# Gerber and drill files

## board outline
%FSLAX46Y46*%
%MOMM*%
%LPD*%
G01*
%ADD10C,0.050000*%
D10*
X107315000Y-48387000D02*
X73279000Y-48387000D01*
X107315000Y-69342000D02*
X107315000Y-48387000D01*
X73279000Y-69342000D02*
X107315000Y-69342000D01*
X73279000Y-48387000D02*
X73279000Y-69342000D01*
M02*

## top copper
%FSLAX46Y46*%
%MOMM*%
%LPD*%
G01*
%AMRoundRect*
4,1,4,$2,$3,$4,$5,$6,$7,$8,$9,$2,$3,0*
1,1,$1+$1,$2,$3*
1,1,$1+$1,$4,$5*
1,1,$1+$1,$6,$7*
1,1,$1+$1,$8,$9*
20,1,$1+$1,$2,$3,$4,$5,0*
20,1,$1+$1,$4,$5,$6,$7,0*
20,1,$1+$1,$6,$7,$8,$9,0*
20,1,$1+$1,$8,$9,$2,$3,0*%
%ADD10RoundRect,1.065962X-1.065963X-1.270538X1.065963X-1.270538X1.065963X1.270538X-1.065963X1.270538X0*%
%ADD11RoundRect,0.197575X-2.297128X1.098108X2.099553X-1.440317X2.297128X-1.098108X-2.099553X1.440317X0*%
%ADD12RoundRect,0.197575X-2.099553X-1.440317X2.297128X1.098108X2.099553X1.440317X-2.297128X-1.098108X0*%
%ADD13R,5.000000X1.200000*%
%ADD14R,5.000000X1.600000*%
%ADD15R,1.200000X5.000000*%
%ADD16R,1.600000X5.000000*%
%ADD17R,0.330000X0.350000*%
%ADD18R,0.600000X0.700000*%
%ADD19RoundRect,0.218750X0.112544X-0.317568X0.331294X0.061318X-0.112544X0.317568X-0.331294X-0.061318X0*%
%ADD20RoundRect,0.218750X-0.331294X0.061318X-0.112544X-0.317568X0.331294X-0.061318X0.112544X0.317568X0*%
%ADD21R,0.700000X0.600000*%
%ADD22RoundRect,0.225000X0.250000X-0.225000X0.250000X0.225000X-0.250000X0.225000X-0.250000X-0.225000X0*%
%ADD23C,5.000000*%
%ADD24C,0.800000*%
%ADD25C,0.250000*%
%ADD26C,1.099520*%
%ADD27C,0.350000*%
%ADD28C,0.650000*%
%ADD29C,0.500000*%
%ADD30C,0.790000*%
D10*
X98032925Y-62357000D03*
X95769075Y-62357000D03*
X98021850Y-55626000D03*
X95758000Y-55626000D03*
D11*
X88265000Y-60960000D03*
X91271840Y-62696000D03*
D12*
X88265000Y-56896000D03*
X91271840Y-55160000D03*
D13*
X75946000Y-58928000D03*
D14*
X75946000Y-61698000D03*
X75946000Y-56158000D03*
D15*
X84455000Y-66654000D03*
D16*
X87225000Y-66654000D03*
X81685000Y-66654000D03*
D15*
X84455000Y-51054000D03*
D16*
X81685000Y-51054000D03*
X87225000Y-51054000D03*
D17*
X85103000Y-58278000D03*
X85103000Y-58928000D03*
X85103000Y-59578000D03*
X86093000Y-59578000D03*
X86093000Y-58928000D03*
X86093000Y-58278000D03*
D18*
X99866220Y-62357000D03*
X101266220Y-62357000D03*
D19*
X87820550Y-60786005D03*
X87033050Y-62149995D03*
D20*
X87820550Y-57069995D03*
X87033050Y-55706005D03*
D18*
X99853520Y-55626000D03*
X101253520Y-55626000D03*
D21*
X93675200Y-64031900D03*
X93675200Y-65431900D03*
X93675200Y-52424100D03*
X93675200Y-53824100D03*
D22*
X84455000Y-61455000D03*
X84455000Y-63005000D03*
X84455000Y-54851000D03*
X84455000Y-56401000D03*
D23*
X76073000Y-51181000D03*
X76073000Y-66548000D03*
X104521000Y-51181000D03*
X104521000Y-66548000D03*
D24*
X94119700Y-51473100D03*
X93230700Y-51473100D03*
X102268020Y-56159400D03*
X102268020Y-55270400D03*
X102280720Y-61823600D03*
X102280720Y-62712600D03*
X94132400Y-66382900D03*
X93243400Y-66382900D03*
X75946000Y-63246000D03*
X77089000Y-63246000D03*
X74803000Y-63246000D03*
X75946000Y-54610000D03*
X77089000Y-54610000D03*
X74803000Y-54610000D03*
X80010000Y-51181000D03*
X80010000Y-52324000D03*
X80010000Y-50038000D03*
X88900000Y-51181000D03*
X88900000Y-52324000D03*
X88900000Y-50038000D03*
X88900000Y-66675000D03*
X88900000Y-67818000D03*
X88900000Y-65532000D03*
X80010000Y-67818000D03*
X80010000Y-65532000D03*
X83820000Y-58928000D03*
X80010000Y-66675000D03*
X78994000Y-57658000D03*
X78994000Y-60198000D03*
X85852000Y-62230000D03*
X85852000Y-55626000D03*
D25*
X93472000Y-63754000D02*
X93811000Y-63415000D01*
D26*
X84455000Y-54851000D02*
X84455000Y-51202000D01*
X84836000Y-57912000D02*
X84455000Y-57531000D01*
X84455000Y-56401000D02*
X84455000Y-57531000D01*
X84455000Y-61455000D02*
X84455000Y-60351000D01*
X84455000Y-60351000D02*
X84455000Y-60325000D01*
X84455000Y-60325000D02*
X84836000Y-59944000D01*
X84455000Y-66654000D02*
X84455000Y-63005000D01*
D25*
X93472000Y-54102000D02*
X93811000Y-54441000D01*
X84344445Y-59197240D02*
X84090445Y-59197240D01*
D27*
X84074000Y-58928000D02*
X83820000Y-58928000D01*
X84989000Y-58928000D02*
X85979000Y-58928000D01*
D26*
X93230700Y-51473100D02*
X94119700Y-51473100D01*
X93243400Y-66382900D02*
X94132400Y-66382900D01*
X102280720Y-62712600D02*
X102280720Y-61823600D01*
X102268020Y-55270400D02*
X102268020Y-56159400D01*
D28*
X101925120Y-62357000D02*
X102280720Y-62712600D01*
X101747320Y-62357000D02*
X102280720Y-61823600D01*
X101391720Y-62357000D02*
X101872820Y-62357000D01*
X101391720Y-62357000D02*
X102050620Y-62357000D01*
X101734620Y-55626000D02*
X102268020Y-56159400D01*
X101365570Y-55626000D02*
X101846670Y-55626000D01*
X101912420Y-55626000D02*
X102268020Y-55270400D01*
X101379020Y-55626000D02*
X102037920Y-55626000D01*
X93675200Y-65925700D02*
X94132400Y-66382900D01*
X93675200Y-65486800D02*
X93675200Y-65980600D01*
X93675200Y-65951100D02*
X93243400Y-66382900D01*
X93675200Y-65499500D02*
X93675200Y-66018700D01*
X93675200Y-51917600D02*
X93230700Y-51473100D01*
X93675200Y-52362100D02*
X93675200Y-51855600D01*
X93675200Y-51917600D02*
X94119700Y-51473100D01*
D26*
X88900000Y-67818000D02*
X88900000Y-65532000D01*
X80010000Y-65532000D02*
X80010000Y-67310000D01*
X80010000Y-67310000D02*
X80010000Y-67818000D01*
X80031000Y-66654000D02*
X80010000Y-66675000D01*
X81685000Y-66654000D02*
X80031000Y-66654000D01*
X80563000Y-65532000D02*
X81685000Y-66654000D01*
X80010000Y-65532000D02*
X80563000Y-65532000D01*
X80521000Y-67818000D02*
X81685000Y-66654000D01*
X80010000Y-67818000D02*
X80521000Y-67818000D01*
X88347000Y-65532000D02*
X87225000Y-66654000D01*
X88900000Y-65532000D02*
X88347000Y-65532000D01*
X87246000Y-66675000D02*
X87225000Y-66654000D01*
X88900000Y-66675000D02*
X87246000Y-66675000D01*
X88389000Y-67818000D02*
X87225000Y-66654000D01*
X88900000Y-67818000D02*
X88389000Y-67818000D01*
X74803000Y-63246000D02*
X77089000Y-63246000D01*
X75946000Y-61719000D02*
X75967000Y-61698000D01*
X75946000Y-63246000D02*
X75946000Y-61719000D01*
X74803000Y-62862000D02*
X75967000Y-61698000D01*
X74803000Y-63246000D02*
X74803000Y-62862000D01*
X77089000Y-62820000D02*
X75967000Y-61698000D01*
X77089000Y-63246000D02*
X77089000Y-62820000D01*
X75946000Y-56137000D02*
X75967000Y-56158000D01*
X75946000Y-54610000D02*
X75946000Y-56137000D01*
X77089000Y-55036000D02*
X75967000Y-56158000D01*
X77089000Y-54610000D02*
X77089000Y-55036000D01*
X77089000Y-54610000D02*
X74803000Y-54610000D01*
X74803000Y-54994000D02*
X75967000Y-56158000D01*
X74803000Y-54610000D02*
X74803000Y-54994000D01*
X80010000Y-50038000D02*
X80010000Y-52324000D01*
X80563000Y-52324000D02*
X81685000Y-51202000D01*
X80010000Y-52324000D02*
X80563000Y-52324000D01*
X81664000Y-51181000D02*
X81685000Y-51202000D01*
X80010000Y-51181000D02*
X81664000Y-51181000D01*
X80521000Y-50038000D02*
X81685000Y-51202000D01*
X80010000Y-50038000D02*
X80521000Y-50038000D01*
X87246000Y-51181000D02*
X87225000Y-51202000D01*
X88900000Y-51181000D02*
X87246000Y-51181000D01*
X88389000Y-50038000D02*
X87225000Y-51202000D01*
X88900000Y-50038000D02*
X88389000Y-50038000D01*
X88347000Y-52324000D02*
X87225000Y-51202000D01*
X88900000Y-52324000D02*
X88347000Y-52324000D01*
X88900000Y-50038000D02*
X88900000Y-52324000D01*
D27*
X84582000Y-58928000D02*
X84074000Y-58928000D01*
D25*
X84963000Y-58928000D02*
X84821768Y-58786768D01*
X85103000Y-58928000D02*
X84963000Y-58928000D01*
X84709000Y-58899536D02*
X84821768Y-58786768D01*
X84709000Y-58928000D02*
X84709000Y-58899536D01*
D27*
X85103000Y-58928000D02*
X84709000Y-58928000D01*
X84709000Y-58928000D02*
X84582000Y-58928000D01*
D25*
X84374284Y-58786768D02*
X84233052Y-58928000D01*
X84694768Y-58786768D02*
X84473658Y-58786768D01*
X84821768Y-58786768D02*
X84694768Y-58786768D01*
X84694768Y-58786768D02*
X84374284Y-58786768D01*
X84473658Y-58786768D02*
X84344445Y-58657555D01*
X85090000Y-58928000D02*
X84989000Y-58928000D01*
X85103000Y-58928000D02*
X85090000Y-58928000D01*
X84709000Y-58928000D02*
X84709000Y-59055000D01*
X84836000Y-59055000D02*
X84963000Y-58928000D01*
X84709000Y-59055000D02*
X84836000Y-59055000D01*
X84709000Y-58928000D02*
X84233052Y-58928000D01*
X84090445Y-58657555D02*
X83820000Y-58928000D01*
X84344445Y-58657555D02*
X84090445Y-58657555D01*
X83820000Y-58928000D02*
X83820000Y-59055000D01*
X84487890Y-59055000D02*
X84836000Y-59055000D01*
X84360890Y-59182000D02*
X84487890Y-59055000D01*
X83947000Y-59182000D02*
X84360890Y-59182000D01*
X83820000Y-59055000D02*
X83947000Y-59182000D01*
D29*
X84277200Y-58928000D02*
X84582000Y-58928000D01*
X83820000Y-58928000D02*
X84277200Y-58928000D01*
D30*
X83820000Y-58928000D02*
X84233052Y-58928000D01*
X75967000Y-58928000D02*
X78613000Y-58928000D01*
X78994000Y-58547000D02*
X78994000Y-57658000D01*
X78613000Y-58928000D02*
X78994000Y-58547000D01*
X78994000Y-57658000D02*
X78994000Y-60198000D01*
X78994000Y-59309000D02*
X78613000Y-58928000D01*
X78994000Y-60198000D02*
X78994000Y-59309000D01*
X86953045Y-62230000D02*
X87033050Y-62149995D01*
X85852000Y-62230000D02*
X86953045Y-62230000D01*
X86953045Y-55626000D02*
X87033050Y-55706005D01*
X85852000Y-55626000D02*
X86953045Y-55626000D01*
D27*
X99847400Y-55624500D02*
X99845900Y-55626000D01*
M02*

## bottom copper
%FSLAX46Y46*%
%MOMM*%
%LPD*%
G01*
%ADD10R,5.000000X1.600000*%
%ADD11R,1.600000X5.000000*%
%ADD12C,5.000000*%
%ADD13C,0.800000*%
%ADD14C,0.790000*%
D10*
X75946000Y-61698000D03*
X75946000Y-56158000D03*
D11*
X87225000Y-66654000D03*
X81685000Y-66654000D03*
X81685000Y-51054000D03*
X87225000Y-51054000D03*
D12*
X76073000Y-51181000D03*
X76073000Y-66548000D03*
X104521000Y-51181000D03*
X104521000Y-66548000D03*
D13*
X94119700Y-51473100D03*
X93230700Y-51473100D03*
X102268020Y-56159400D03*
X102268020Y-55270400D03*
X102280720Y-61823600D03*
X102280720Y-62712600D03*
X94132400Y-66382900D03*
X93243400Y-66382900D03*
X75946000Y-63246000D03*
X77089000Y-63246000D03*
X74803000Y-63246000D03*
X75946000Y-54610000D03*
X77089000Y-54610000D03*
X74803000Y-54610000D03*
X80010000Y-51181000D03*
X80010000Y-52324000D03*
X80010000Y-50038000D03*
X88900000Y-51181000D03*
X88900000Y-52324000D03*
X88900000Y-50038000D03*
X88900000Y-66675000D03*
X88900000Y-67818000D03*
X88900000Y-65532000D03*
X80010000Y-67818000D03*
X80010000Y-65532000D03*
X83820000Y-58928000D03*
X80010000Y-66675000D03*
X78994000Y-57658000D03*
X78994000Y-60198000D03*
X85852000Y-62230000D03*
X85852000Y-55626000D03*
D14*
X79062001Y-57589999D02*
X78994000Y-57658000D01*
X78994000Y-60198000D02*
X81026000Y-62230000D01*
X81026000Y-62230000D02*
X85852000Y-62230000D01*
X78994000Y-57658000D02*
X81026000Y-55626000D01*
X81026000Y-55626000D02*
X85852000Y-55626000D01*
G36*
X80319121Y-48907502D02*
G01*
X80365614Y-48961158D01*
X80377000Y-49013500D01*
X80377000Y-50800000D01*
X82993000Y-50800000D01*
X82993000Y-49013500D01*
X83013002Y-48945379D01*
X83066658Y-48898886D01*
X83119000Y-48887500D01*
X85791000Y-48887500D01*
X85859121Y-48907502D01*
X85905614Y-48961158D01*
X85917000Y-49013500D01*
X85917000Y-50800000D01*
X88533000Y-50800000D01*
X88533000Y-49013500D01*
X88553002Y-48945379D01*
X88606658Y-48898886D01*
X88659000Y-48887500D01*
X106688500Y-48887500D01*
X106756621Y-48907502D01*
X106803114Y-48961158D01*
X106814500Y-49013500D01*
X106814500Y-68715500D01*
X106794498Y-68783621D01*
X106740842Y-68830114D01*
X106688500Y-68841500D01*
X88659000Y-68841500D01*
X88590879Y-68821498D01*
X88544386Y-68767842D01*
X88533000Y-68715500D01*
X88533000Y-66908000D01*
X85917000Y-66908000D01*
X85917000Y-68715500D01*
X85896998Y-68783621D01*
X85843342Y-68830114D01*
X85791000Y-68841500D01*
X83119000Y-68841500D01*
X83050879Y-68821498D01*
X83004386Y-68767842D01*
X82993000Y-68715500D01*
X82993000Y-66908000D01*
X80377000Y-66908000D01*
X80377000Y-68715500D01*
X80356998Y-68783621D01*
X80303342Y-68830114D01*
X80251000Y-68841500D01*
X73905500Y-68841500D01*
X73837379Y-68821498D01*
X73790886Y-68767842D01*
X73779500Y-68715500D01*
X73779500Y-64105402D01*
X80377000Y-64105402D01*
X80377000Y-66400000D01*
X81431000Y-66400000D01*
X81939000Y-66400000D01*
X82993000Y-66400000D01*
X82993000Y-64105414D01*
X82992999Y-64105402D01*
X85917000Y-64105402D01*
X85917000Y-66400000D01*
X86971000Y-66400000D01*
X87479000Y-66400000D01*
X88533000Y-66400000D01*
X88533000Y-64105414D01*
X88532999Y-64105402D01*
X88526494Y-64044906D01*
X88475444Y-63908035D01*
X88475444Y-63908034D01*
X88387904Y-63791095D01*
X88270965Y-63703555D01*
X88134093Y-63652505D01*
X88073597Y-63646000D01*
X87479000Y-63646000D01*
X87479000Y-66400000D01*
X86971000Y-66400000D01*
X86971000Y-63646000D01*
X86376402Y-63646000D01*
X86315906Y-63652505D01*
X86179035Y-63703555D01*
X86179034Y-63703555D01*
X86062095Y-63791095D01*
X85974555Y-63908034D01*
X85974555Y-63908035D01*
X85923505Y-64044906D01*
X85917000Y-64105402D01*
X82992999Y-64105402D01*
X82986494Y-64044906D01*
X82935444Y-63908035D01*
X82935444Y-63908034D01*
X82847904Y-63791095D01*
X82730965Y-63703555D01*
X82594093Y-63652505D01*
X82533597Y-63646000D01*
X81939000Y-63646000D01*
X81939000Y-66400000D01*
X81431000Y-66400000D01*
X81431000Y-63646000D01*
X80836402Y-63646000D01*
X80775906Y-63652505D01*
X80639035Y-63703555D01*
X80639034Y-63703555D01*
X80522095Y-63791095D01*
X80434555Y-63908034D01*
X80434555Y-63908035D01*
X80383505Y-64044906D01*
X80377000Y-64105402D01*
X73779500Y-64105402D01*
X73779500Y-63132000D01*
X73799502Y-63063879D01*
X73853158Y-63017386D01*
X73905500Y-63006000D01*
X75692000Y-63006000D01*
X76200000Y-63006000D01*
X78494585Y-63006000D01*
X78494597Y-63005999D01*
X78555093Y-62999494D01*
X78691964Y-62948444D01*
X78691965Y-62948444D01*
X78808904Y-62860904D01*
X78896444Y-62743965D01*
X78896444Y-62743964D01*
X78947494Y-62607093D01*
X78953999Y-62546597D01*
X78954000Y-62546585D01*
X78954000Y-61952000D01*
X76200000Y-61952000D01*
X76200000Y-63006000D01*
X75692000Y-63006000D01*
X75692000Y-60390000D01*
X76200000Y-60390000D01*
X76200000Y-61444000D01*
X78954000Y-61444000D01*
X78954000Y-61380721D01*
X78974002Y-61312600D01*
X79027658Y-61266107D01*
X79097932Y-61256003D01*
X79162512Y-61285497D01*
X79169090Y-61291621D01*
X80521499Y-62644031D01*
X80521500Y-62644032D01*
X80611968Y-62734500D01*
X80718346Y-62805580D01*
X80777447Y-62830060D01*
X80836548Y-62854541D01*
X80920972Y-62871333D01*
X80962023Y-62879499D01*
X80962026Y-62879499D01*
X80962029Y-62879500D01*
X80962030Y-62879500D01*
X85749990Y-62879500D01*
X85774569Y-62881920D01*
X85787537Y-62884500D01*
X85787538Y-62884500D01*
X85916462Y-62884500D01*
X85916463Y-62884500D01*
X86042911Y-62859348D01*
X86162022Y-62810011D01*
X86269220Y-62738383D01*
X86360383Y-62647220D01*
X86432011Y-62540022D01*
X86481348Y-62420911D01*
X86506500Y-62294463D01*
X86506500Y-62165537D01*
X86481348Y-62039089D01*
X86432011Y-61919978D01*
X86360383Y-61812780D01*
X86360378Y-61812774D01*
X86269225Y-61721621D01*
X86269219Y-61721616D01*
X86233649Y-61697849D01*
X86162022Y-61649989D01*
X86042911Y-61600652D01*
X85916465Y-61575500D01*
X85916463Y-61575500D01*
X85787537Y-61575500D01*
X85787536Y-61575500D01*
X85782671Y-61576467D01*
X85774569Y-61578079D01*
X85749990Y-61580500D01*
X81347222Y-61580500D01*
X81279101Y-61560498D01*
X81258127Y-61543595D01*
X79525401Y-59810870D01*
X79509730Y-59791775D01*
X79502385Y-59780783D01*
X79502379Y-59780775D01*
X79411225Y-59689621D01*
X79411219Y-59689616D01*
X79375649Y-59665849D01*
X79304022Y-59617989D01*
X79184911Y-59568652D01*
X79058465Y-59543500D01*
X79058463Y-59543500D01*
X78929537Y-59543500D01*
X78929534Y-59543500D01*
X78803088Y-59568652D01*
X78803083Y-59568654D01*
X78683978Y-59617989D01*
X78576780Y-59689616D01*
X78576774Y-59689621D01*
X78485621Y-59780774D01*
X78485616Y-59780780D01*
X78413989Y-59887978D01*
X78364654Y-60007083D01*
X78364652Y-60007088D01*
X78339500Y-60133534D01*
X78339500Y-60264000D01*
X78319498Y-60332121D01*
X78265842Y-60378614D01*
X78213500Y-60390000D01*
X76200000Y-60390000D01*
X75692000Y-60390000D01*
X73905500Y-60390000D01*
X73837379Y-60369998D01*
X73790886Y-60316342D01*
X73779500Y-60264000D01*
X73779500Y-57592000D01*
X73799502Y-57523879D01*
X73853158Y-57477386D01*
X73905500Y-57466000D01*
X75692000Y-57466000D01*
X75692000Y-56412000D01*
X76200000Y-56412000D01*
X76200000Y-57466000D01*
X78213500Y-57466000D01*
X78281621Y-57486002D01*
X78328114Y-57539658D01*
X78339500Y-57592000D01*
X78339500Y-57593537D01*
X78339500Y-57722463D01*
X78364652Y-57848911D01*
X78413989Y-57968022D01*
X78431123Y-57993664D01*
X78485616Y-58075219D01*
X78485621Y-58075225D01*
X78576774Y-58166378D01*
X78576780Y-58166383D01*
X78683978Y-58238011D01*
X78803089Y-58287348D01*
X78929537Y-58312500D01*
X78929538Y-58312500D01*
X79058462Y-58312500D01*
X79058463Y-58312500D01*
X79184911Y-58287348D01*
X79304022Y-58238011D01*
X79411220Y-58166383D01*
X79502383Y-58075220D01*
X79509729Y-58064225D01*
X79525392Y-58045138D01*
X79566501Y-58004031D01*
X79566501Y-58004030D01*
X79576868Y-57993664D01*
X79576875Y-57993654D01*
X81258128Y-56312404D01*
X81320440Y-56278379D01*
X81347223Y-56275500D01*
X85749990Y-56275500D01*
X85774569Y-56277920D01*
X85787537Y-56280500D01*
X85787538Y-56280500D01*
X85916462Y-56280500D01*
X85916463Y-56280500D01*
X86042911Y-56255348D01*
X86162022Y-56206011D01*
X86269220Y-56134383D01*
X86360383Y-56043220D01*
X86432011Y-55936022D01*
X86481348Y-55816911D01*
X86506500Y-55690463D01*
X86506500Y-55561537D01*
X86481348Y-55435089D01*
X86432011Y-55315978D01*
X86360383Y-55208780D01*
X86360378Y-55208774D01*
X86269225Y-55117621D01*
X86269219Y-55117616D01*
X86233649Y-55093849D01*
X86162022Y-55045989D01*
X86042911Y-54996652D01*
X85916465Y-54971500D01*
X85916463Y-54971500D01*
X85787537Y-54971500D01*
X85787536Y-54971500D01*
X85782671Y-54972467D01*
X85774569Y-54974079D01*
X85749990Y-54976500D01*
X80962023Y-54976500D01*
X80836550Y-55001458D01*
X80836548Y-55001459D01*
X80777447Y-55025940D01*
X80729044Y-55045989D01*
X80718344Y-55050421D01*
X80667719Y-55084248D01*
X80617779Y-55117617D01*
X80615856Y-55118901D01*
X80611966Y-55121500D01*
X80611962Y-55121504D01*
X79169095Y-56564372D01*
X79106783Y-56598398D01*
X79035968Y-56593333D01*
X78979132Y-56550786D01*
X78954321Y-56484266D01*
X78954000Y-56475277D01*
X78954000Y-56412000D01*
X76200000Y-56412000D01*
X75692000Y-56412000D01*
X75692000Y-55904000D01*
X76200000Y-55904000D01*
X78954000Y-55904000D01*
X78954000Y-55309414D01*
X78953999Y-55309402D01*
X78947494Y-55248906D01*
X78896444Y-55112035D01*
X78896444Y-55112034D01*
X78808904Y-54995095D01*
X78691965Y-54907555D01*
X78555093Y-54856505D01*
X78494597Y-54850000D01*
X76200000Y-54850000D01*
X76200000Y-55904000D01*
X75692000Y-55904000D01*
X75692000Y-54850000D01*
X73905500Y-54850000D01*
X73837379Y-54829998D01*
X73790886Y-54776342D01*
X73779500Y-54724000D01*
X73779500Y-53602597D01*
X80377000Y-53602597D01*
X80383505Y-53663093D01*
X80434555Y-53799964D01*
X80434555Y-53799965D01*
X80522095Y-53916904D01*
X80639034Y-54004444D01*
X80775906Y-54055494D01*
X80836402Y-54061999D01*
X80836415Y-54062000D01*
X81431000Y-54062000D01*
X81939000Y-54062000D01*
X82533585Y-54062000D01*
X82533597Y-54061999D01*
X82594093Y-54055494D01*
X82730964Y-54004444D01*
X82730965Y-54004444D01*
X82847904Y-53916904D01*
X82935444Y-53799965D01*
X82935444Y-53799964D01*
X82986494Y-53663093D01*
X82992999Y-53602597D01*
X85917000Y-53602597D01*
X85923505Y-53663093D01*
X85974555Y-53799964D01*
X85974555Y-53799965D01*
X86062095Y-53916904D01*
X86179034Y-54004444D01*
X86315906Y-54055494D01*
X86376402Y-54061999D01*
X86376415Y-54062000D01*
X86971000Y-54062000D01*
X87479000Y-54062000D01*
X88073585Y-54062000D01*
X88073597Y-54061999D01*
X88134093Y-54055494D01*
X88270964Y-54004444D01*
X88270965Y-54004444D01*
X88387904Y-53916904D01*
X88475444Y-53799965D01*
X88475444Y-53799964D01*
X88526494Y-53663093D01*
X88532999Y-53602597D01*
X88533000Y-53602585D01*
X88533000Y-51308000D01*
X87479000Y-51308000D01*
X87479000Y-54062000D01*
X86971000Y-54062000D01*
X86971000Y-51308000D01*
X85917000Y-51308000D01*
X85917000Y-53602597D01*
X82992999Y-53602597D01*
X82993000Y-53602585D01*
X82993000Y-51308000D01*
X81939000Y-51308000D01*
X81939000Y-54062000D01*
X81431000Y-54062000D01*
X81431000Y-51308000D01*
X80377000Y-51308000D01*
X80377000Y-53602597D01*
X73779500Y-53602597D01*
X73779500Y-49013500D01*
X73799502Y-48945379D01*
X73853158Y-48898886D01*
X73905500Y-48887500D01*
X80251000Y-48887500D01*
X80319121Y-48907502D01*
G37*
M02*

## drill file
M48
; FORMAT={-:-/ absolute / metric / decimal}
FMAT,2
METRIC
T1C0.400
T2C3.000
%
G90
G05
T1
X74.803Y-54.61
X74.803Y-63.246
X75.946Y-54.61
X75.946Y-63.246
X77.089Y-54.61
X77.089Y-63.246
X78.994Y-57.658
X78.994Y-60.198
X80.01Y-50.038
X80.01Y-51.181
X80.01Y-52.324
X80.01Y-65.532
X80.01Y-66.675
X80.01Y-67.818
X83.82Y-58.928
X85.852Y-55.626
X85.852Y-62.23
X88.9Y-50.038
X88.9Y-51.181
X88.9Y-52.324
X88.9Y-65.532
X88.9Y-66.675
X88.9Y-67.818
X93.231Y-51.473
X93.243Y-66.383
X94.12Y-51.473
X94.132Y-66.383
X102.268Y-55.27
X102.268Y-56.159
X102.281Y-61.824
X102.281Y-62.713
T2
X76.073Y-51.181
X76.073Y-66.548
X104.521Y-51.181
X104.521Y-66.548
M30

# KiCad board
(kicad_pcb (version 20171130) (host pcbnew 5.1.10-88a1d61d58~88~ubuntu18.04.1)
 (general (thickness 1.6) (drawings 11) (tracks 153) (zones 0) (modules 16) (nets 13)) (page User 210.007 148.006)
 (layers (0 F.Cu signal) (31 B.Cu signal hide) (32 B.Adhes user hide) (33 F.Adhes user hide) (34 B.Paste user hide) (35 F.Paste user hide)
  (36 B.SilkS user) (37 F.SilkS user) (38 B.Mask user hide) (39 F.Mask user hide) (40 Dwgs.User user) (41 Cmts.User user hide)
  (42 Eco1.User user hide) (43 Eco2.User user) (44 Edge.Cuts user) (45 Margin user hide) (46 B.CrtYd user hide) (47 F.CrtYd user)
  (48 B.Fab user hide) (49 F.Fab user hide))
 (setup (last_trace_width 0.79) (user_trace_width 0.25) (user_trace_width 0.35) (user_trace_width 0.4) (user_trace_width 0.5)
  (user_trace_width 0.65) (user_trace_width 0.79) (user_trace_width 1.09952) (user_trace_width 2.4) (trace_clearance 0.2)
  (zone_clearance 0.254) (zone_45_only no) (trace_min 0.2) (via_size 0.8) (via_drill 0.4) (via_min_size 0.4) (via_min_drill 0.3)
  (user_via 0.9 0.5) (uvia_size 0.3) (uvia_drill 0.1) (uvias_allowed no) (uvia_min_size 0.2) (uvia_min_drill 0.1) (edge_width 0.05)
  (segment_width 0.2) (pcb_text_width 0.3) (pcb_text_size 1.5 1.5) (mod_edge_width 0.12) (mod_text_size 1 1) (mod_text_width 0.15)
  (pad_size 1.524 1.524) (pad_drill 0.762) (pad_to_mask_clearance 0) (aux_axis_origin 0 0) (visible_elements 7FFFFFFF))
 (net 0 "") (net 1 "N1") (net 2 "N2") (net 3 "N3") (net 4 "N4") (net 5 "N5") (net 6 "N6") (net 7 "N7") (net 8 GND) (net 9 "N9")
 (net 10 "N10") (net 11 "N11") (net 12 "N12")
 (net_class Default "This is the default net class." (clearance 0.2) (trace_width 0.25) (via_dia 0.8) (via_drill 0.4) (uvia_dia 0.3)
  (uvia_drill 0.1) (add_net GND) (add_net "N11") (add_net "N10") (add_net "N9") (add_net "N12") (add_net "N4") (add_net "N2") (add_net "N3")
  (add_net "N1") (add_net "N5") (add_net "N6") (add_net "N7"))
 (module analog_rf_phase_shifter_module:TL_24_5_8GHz (layer F.Cu) (at 96.901 62.357)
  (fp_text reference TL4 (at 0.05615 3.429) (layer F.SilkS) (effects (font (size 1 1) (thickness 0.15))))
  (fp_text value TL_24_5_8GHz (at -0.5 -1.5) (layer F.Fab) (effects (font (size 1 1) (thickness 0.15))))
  (pad 2 smd roundrect (at 1.131925 0) (size 4.26385 4.673) (layers F.Cu) (roundrect_rratio 0.2499998827350868) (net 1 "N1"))
  (pad 1 smd roundrect (at -1.131925 0) (size 4.26385 4.673) (layers F.Cu) (roundrect_rratio 0.2499998827350868) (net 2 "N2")))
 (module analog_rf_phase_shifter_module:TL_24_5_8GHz (layer F.Cu) (at 96.889925 55.626)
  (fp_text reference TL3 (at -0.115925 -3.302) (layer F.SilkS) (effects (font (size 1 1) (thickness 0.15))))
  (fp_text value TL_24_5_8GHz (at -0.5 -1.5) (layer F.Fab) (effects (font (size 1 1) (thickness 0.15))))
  (pad 2 smd roundrect (at 1.131925 0) (size 4.26385 4.673) (layers F.Cu) (roundrect_rratio 0.2499998827350868) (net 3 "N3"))
  (pad 1 smd roundrect (at -1.131925 0) (size 4.26385 4.673) (layers F.Cu) (roundrect_rratio 0.2499998827350868) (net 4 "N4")))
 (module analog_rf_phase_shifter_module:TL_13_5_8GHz (layer F.Cu) (at 89.76842 61.828 330)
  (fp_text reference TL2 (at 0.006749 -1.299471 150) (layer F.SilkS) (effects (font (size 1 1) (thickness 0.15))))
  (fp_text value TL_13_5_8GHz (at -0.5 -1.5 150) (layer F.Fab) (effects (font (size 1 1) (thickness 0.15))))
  (pad 1 smd roundrect (at -1.736 0 330) (size 5.472 0.7903) (layers F.Cu) (roundrect_rratio 0.25) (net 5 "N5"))
  (pad 2 smd roundrect (at 1.736 0 330) (size 5.472 0.7903) (layers F.Cu) (roundrect_rratio 0.25) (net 2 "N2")))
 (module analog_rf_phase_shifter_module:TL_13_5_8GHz (layer F.Cu) (at 89.76842 56.028 30)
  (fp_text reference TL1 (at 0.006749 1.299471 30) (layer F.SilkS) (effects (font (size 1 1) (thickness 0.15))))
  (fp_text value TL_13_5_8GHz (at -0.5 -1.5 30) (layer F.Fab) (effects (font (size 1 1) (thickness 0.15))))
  (pad 1 smd roundrect (at -1.736 0 30) (size 5.472 0.7903) (layers F.Cu) (roundrect_rratio 0.25) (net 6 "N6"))
  (pad 2 smd roundrect (at 1.736 0 30) (size 5.472 0.7903) (layers F.Cu) (roundrect_rratio 0.25) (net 4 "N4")))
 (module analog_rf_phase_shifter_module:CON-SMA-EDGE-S (layer F.Cu) (at 68.686 58.928 90)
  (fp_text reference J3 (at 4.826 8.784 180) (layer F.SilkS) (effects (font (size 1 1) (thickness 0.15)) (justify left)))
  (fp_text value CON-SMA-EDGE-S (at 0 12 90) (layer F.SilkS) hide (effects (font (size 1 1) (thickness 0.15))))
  (pad 1 smd rect (at 0 7.26 90) (size 1.2 5) (layers F.Cu F.Paste F.Mask) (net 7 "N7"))
  (pad 2 smd rect (at -2.77 7.26 90) (size 1.6 5) (layers F.Cu F.Paste F.Mask) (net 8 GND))
  (pad 2 smd rect (at 2.77 7.26 90) (size 1.6 5) (layers F.Cu F.Paste F.Mask) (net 8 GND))
  (pad 2 smd rect (at -2.77 7.26 90) (size 1.6 5) (layers B.Cu B.Paste B.Mask) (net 8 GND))
  (pad 2 smd rect (at 2.77 7.26 90) (size 1.6 5) (layers B.Cu B.Paste B.Mask) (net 8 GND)))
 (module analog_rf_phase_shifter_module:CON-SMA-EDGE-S (layer F.Cu) (at 84.455 73.914 180)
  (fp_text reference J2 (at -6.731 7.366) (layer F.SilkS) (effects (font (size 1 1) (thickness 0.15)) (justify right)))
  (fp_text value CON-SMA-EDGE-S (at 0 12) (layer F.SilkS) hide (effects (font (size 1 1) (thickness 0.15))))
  (pad 1 smd rect (at 0 7.26 180) (size 1.2 5) (layers F.Cu F.Paste F.Mask) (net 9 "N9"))
  (pad 2 smd rect (at -2.77 7.26 180) (size 1.6 5) (layers F.Cu F.Paste F.Mask) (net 8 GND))
  (pad 2 smd rect (at 2.77 7.26 180) (size 1.6 5) (layers F.Cu F.Paste F.Mask) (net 8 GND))
  (pad 2 smd rect (at -2.77 7.26 180) (size 1.6 5) (layers B.Cu B.Paste B.Mask) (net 8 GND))
  (pad 2 smd rect (at 2.77 7.26 180) (size 1.6 5) (layers B.Cu B.Paste B.Mask) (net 8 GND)))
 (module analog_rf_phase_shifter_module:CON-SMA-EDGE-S (layer F.Cu) (at 84.455 43.794)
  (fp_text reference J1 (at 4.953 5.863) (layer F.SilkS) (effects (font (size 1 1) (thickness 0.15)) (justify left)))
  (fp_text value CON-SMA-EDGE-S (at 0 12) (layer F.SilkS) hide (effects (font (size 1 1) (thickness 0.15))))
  (pad 1 smd rect (at 0 7.26) (size 1.2 5) (layers F.Cu F.Paste F.Mask) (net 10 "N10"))
  (pad 2 smd rect (at -2.77 7.26) (size 1.6 5) (layers F.Cu F.Paste F.Mask) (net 8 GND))
  (pad 2 smd rect (at 2.77 7.26) (size 1.6 5) (layers F.Cu F.Paste F.Mask) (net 8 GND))
  (pad 2 smd rect (at -2.77 7.26) (size 1.6 5) (layers B.Cu B.Paste B.Mask) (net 8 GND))
  (pad 2 smd rect (at 2.77 7.26) (size 1.6 5) (layers B.Cu B.Paste B.Mask) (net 8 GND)))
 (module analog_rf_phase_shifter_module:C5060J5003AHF (layer F.Cu) (at 85.598 58.928 270)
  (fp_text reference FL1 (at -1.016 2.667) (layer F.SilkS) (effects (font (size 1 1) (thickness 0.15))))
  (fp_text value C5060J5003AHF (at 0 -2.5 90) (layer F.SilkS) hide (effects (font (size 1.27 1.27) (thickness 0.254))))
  (pad 1 smd rect (at -0.65 0.495) (size 0.33 0.35) (layers F.Cu F.Paste F.Mask) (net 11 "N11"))
  (pad 2 smd rect (at 0 0.495) (size 0.33 0.35) (layers F.Cu F.Paste F.Mask) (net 8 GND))
  (pad 3 smd rect (at 0.65 0.495) (size 0.33 0.35) (layers F.Cu F.Paste F.Mask) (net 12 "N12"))
  (pad 4 smd rect (at 0.65 -0.495) (size 0.33 0.35) (layers F.Cu F.Paste F.Mask) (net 5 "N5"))
  (pad 5 smd rect (at 0 -0.495) (size 0.33 0.35) (layers F.Cu F.Paste F.Mask) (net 8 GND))
  (pad 6 smd rect (at -0.65 -0.495) (size 0.33 0.35) (layers F.Cu F.Paste F.Mask) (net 6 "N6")))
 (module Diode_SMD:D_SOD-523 (layer F.Cu) (at 100.56622 62.357)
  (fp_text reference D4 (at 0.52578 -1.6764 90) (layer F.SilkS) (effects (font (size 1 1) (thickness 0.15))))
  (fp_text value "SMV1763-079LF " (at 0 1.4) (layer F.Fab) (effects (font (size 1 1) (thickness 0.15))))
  (pad 1 smd rect (at -0.7 0 180) (size 0.6 0.7) (layers F.Cu F.Paste F.Mask) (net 1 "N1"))
  (pad 2 smd rect (at 0.7 0 180) (size 0.6 0.7) (layers F.Cu F.Paste F.Mask) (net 8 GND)))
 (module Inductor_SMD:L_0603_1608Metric (layer F.Cu) (at 87.4268 61.468 60)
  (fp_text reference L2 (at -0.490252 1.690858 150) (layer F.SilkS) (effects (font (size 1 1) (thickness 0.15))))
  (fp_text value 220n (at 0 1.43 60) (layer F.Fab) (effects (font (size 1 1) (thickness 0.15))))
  (pad 2 smd roundrect (at 0.7875 0 60) (size 0.875 0.95) (layers F.Cu F.Paste F.Mask) (roundrect_rratio 0.25) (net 5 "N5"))
  (pad 1 smd roundrect (at -0.7875 0 60) (size 0.875 0.95) (layers F.Cu F.Paste F.Mask) (roundrect_rratio 0.25) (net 7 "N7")))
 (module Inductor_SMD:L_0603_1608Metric (layer F.Cu) (at 87.4268 56.388 300)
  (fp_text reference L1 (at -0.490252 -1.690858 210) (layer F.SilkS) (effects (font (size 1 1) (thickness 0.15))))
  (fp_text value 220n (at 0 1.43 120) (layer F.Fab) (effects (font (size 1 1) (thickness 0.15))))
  (pad 2 smd roundrect (at 0.7875 0 300) (size 0.875 0.95) (layers F.Cu F.Paste F.Mask) (roundrect_rratio 0.25) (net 6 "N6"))
  (pad 1 smd roundrect (at -0.7875 0 300) (size 0.875 0.95) (layers F.Cu F.Paste F.Mask) (roundrect_rratio 0.25) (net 7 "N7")))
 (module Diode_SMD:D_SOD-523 (layer F.Cu) (at 100.55352 55.626)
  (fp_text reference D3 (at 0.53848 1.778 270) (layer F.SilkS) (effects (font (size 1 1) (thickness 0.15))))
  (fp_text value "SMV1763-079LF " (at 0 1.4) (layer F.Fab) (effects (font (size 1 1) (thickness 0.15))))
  (pad 1 smd rect (at -0.7 0 180) (size 0.6 0.7) (layers F.Cu F.Paste F.Mask) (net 3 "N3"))
  (pad 2 smd rect (at 0.7 0 180) (size 0.6 0.7) (layers F.Cu F.Paste F.Mask) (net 8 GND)))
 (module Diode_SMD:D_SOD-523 (layer F.Cu) (at 93.6752 64.7319 270)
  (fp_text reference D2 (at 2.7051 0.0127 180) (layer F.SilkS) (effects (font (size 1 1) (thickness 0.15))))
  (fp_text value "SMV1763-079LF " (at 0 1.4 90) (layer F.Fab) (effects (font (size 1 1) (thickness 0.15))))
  (pad 1 smd rect (at -0.7 0 90) (size 0.6 0.7) (layers F.Cu F.Paste F.Mask) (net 2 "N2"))
  (pad 2 smd rect (at 0.7 0 90) (size 0.6 0.7) (layers F.Cu F.Paste F.Mask) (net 8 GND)))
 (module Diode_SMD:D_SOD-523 (layer F.Cu) (at 93.6752 53.1241 90)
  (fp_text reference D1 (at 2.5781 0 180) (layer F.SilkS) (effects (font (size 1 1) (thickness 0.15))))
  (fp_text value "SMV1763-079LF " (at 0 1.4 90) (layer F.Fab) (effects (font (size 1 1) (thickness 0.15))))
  (pad 2 smd rect (at 0.7 0 270) (size 0.6 0.7) (layers F.Cu F.Paste F.Mask) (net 8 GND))
  (pad 1 smd rect (at -0.7 0 270) (size 0.6 0.7) (layers F.Cu F.Paste F.Mask) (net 4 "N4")))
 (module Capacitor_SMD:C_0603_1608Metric (layer F.Cu) (at 84.455 62.23 90)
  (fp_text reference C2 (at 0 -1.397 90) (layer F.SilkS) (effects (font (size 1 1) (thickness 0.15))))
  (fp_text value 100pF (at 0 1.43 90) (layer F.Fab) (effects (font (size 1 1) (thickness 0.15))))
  (pad 2 smd roundrect (at 0.775 0 90) (size 0.9 0.95) (layers F.Cu F.Paste F.Mask) (roundrect_rratio 0.25) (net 12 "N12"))
  (pad 1 smd roundrect (at -0.775 0 90) (size 0.9 0.95) (layers F.Cu F.Paste F.Mask) (roundrect_rratio 0.25) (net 9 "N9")))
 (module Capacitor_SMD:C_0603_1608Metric (layer F.Cu) (at 84.455 55.626 90)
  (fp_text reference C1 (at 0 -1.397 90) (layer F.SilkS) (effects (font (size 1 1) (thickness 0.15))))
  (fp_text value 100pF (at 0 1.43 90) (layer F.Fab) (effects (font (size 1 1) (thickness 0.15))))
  (pad 2 smd roundrect (at 0.775 0 90) (size 0.9 0.95) (layers F.Cu F.Paste F.Mask) (roundrect_rratio 0.25) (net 10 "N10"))
  (pad 1 smd roundrect (at -0.775 0 90) (size 0.9 0.95) (layers F.Cu F.Paste F.Mask) (roundrect_rratio 0.25) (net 11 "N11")))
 (gr_line (start 107.315 48.387) (end 73.279 48.387) (layer Edge.Cuts) (width 0.05))
 (gr_line (start 107.315 69.342) (end 107.315 48.387) (layer Edge.Cuts) (width 0.05))
 (gr_line (start 73.279 69.342) (end 107.315 69.342) (layer Edge.Cuts) (width 0.05))
 (gr_line (start 73.279 48.387) (end 73.279 69.342) (layer Edge.Cuts) (width 0.05))
 (segment (start 93.472 63.754) (end 93.811 63.415) (width 0.25) (layer F.Cu) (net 2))
 (segment (start 84.455 54.851) (end 84.455 51.202) (width 1.09952) (layer F.Cu) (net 10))
 (segment (start 84.836 57.912) (end 84.455 57.531) (width 1.09952) (layer F.Cu) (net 11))
 (segment (start 84.455 56.401) (end 84.455 57.531) (width 1.09952) (layer F.Cu) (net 11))
 (segment (start 84.455 61.455) (end 84.455 60.351) (width 1.09952) (layer F.Cu) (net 12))
 (segment (start 84.455 60.351) (end 84.455 60.325) (width 1.09952) (layer F.Cu) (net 12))
 (segment (start 84.455 60.325) (end 84.836 59.944) (width 1.09952) (layer F.Cu) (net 12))
 (segment (start 84.455 66.654) (end 84.455 63.005) (width 1.09952) (layer F.Cu) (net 9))
 (segment (start 93.472 54.102) (end 93.811 54.441) (width 0.25) (layer F.Cu) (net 4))
 (segment (start 84.344445 59.19724) (end 84.090445 59.19724) (width 0.25) (layer F.Cu) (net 8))
 (via (at 76.073 51.181) (size 5) (drill 3) (layers F.Cu B.Cu) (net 8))
 (via (at 76.073 66.548) (size 5) (drill 3) (layers F.Cu B.Cu) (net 8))
 (via (at 104.521 51.181) (size 5) (drill 3) (layers F.Cu B.Cu) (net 8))
 (via (at 104.521 66.548) (size 5) (drill 3) (layers F.Cu B.Cu) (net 8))
 (via (at 94.1197 51.4731) (size 0.8) (drill 0.4) (layers F.Cu B.Cu) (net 8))
 (via (at 93.2307 51.4731) (size 0.8) (drill 0.4) (layers F.Cu B.Cu) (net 8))
 (via (at 102.26802 56.1594) (size 0.8) (drill 0.4) (layers F.Cu B.Cu) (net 8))
 (via (at 102.26802 55.2704) (size 0.8) (drill 0.4) (layers F.Cu B.Cu) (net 8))
 (via (at 102.28072 61.8236) (size 0.8) (drill 0.4) (layers F.Cu B.Cu) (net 8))
 (via (at 102.28072 62.7126) (size 0.8) (drill 0.4) (layers F.Cu B.Cu) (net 8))
 (via (at 94.1324 66.3829) (size 0.8) (drill 0.4) (layers F.Cu B.Cu) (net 8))
 (via (at 93.2434 66.3829) (size 0.8) (drill 0.4) (layers F.Cu B.Cu) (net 8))
 (via (at 75.946 63.246) (size 0.8) (drill 0.4) (layers F.Cu B.Cu) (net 8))
 (via (at 77.089 63.246) (size 0.8) (drill 0.4) (layers F.Cu B.Cu) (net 8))
 (via (at 74.803 63.246) (size 0.8) (drill 0.4) (layers F.Cu B.Cu) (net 8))
 (via (at 75.946 54.61) (size 0.8) (drill 0.4) (layers F.Cu B.Cu) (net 8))
 (via (at 77.089 54.61) (size 0.8) (drill 0.4) (layers F.Cu B.Cu) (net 8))
 (via (at 74.803 54.61) (size 0.8) (drill 0.4) (layers F.Cu B.Cu) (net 8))
 (via (at 80.01 51.181) (size 0.8) (drill 0.4) (layers F.Cu B.Cu) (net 8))
 (via (at 80.01 52.324) (size 0.8) (drill 0.4) (layers F.Cu B.Cu) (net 8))
 (via (at 80.01 50.038) (size 0.8) (drill 0.4) (layers F.Cu B.Cu) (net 8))
 (via (at 88.9 51.181) (size 0.8) (drill 0.4) (layers F.Cu B.Cu) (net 8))
 (via (at 88.9 52.324) (size 0.8) (drill 0.4) (layers F.Cu B.Cu) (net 8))
 (via (at 88.9 50.038) (size 0.8) (drill 0.4) (layers F.Cu B.Cu) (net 8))
 (via (at 88.9 66.675) (size 0.8) (drill 0.4) (layers F.Cu B.Cu) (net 8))
 (via (at 88.9 67.818) (size 0.8) (drill 0.4) (layers F.Cu B.Cu) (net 8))
 (via (at 88.9 65.532) (size 0.8) (drill 0.4) (layers F.Cu B.Cu) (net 8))
 (via (at 80.01 67.818) (size 0.8) (drill 0.4) (layers F.Cu B.Cu) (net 8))
 (via (at 80.01 65.532) (size 0.8) (drill 0.4) (layers F.Cu B.Cu) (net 8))
 (via (at 83.82 58.928) (size 0.8) (drill 0.4) (layers F.Cu B.Cu) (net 8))
 (segment (start 84.074 58.928) (end 83.82 58.928) (width 0.35) (layer F.Cu) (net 8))
 (segment (start 84.989 58.928) (end 85.979 58.928) (width 0.35) (layer F.Cu) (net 8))
 (via (at 80.01 66.675) (size 0.8) (drill 0.4) (layers F.Cu B.Cu) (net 8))
 (segment (start 93.2307 51.4731) (end 94.1197 51.4731) (width 1.09952) (layer F.Cu) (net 8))
 (segment (start 93.2434 66.3829) (end 94.1324 66.3829) (width 1.09952) (layer F.Cu) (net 8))
 (segment (start 102.28072 62.7126) (end 102.28072 61.8236) (width 1.09952) (layer F.Cu) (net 8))
 (segment (start 102.26802 55.2704) (end 102.26802 56.1594) (width 1.09952) (layer F.Cu) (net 8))
 (segment (start 101.92512 62.357) (end 102.28072 62.7126) (width 0.65) (layer F.Cu) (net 8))
 (segment (start 101.74732 62.357) (end 102.28072 61.8236) (width 0.65) (layer F.Cu) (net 8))
 (segment (start 101.39172 62.357) (end 101.87282 62.357) (width 0.65) (layer F.Cu) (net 8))
 (segment (start 101.39172 62.357) (end 102.05062 62.357) (width 0.65) (layer F.Cu) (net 8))
 (segment (start 101.73462 55.626) (end 102.26802 56.1594) (width 0.65) (layer F.Cu) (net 8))
 (segment (start 101.36557 55.626) (end 101.84667 55.626) (width 0.65) (layer F.Cu) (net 8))
 (segment (start 101.91242 55.626) (end 102.26802 55.2704) (width 0.65) (layer F.Cu) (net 8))
 (segment (start 101.37902 55.626) (end 102.03792 55.626) (width 0.65) (layer F.Cu) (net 8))
 (segment (start 93.6752 65.9257) (end 94.1324 66.3829) (width 0.65) (layer F.Cu) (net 8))
 (segment (start 93.6752 65.4868) (end 93.6752 65.9806) (width 0.65) (layer F.Cu) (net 8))
 (segment (start 93.6752 65.9511) (end 93.2434 66.3829) (width 0.65) (layer F.Cu) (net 8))
 (segment (start 93.6752 65.4995) (end 93.6752 66.0187) (width 0.65) (layer F.Cu) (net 8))
 (segment (start 93.6752 51.9176) (end 93.2307 51.4731) (width 0.65) (layer F.Cu) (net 8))
 (segment (start 93.6752 52.3621) (end 93.6752 51.8556) (width 0.65) (layer F.Cu) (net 8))
 (segment (start 93.6752 51.9176) (end 94.1197 51.4731) (width 0.65) (layer F.Cu) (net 8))
 (segment (start 88.9 67.818) (end 88.9 65.532) (width 1.09952) (layer F.Cu) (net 8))
 (segment (start 80.01 65.532) (end 80.01 67.31) (width 1.09952) (layer F.Cu) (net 8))
 (segment (start 80.01 67.31) (end 80.01 67.818) (width 1.09952) (layer F.Cu) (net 8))
 (segment (start 80.031 66.654) (end 80.01 66.675) (width 1.09952) (layer F.Cu) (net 8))
 (segment (start 81.685 66.654) (end 80.031 66.654) (width 1.09952) (layer F.Cu) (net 8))
 (segment (start 80.563 65.532) (end 81.685 66.654) (width 1.09952) (layer F.Cu) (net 8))
 (segment (start 80.01 65.532) (end 80.563 65.532) (width 1.09952) (layer F.Cu) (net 8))
 (segment (start 80.521 67.818) (end 81.685 66.654) (width 1.09952) (layer F.Cu) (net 8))
 (segment (start 80.01 67.818) (end 80.521 67.818) (width 1.09952) (layer F.Cu) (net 8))
 (segment (start 88.347 65.532) (end 87.225 66.654) (width 1.09952) (layer F.Cu) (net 8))
 (segment (start 88.9 65.532) (end 88.347 65.532) (width 1.09952) (layer F.Cu) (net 8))
 (segment (start 87.246 66.675) (end 87.225 66.654) (width 1.09952) (layer F.Cu) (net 8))
 (segment (start 88.9 66.675) (end 87.246 66.675) (width 1.09952) (layer F.Cu) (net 8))
 (segment (start 88.389 67.818) (end 87.225 66.654) (width 1.09952) (layer F.Cu) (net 8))
 (segment (start 88.9 67.818) (end 88.389 67.818) (width 1.09952) (layer F.Cu) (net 8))
 (segment (start 74.803 63.246) (end 77.089 63.246) (width 1.09952) (layer F.Cu) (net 8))
 (segment (start 75.946 61.719) (end 75.967 61.698) (width 1.09952) (layer F.Cu) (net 8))
 (segment (start 75.946 63.246) (end 75.946 61.719) (width 1.09952) (layer F.Cu) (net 8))
 (segment (start 74.803 62.862) (end 75.967 61.698) (width 1.09952) (layer F.Cu) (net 8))
 (segment (start 74.803 63.246) (end 74.803 62.862) (width 1.09952) (layer F.Cu) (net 8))
 (segment (start 77.089 62.82) (end 75.967 61.698) (width 1.09952) (layer F.Cu) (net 8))
 (segment (start 77.089 63.246) (end 77.089 62.82) (width 1.09952) (layer F.Cu) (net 8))
 (segment (start 75.946 56.137) (end 75.967 56.158) (width 1.09952) (layer F.Cu) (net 8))
 (segment (start 75.946 54.61) (end 75.946 56.137) (width 1.09952) (layer F.Cu) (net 8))
 (segment (start 77.089 55.036) (end 75.967 56.158) (width 1.09952) (layer F.Cu) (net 8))
 (segment (start 77.089 54.61) (end 77.089 55.036) (width 1.09952) (layer F.Cu) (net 8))
 (segment (start 77.089 54.61) (end 74.803 54.61) (width 1.09952) (layer F.Cu) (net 8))
 (segment (start 74.803 54.994) (end 75.967 56.158) (width 1.09952) (layer F.Cu) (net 8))
 (segment (start 74.803 54.61) (end 74.803 54.994) (width 1.09952) (layer F.Cu) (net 8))
 (segment (start 80.01 50.038) (end 80.01 52.324) (width 1.09952) (layer F.Cu) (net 8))
 (segment (start 80.563 52.324) (end 81.685 51.202) (width 1.09952) (layer F.Cu) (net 8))
 (segment (start 80.01 52.324) (end 80.563 52.324) (width 1.09952) (layer F.Cu) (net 8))
 (segment (start 81.664 51.181) (end 81.685 51.202) (width 1.09952) (layer F.Cu) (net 8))
 (segment (start 80.01 51.181) (end 81.664 51.181) (width 1.09952) (layer F.Cu) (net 8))
 (segment (start 80.521 50.038) (end 81.685 51.202) (width 1.09952) (layer F.Cu) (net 8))
 (segment (start 80.01 50.038) (end 80.521 50.038) (width 1.09952) (layer F.Cu) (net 8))
 (segment (start 87.246 51.181) (end 87.225 51.202) (width 1.09952) (layer F.Cu) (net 8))
 (segment (start 88.9 51.181) (end 87.246 51.181) (width 1.09952) (layer F.Cu) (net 8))
 (segment (start 88.389 50.038) (end 87.225 51.202) (width 1.09952) (layer F.Cu) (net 8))
 (segment (start 88.9 50.038) (end 88.389 50.038) (width 1.09952) (layer F.Cu) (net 8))
 (segment (start 88.347 52.324) (end 87.225 51.202) (width 1.09952) (layer F.Cu) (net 8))
 (segment (start 88.9 52.324) (end 88.347 52.324) (width 1.09952) (layer F.Cu) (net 8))
 (segment (start 88.9 50.038) (end 88.9 52.324) (width 1.09952) (layer F.Cu) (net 8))
 (segment (start 84.582 58.928) (end 84.074 58.928) (width 0.35) (layer F.Cu) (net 8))
 (segment (start 84.963 58.928) (end 84.821768 58.786768) (width 0.25) (layer F.Cu) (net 8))
 (segment (start 85.103 58.928) (end 84.963 58.928) (width 0.25) (layer F.Cu) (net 8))
 (segment (start 84.709 58.899536) (end 84.821768 58.786768) (width 0.25) (layer F.Cu) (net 8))
 (segment (start 84.709 58.928) (end 84.709 58.899536) (width 0.25) (layer F.Cu) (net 8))
 (segment (start 85.103 58.928) (end 84.709 58.928) (width 0.35) (layer F.Cu) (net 8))
 (segment (start 84.709 58.928) (end 84.582 58.928) (width 0.35) (layer F.Cu) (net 8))
 (segment (start 84.374284 58.786768) (end 84.233052 58.928) (width 0.25) (layer F.Cu) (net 8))
 (segment (start 84.694768 58.786768) (end 84.473658 58.786768) (width 0.25) (layer F.Cu) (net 8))
 (segment (start 84.821768 58.786768) (end 84.694768 58.786768) (width 0.25) (layer F.Cu) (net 8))
 (segment (start 84.694768 58.786768) (end 84.374284 58.786768) (width 0.25) (layer F.Cu) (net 8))
 (segment (start 84.473658 58.786768) (end 84.344445 58.657555) (width 0.25) (layer F.Cu) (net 8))
 (segment (start 85.09 58.928) (end 84.989 58.928) (width 0.25) (layer F.Cu) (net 8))
 (segment (start 85.103 58.928) (end 85.09 58.928) (width 0.25) (layer F.Cu) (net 8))
 (segment (start 84.709 58.928) (end 84.709 59.055) (width 0.25) (layer F.Cu) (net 8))
 (segment (start 84.836 59.055) (end 84.963 58.928) (width 0.25) (layer F.Cu) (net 8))
 (segment (start 84.709 59.055) (end 84.836 59.055) (width 0.25) (layer F.Cu) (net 8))
 (segment (start 84.709 58.928) (end 84.233052 58.928) (width 0.25) (layer F.Cu) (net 8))
 (segment (start 84.090445 58.657555) (end 83.82 58.928) (width 0.25) (layer F.Cu) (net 8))
 (segment (start 84.344445 58.657555) (end 84.090445 58.657555) (width 0.25) (layer F.Cu) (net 8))
 (segment (start 83.82 58.928) (end 83.82 59.055) (width 0.25) (layer F.Cu) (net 8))
 (segment (start 84.48789 59.055) (end 84.836 59.055) (width 0.25) (layer F.Cu) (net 8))
 (segment (start 84.36089 59.182) (end 84.48789 59.055) (width 0.25) (layer F.Cu) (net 8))
 (segment (start 83.947 59.182) (end 84.36089 59.182) (width 0.25) (layer F.Cu) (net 8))
 (segment (start 83.82 59.055) (end 83.947 59.182) (width 0.25) (layer F.Cu) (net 8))
 (segment (start 84.2772 58.928) (end 84.582 58.928) (width 0.5) (layer F.Cu) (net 8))
 (segment (start 83.82 58.928) (end 84.2772 58.928) (width 0.5) (layer F.Cu) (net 8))
 (segment (start 83.82 58.928) (end 84.233052 58.928) (width 0.79) (layer F.Cu) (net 8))
 (via (at 78.994 57.658) (size 0.8) (drill 0.4) (layers F.Cu B.Cu) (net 7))
 (segment (start 79.062001 57.589999) (end 78.994 57.658) (width 0.79) (layer B.Cu) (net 7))
 (via (at 78.994 60.198) (size 0.8) (drill 0.4) (layers F.Cu B.Cu) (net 7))
 (segment (start 75.967 58.928) (end 78.613 58.928) (width 0.79) (layer F.Cu) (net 7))
 (segment (start 78.994 58.547) (end 78.994 57.658) (width 0.79) (layer F.Cu) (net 7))
 (segment (start 78.613 58.928) (end 78.994 58.547) (width 0.79) (layer F.Cu) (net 7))
 (segment (start 78.994 57.658) (end 78.994 60.198) (width 0.79) (layer F.Cu) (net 7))
 (segment (start 78.994 59.309) (end 78.613 58.928) (width 0.79) (layer F.Cu) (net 7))
 (segment (start 78.994 60.198) (end 78.994 59.309) (width 0.79) (layer F.Cu) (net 7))
 (via (at 85.852 62.23) (size 0.8) (drill 0.4) (layers F.Cu B.Cu) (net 7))
 (segment (start 78.994 60.198) (end 81.026 62.23) (width 0.79) (layer B.Cu) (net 7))
 (segment (start 81.026 62.23) (end 85.852 62.23) (width 0.79) (layer B.Cu) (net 7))
 (segment (start 86.953045 62.23) (end 87.03305 62.149995) (width 0.79) (layer F.Cu) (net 7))
 (segment (start 85.852 62.23) (end 86.953045 62.23) (width 0.79) (layer F.Cu) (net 7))
 (via (at 85.852 55.626) (size 0.8) (drill 0.4) (layers F.Cu B.Cu) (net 7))
 (segment (start 78.994 57.658) (end 81.026 55.626) (width 0.79) (layer B.Cu) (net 7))
 (segment (start 81.026 55.626) (end 85.852 55.626) (width 0.79) (layer B.Cu) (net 7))
 (segment (start 86.953045 55.626) (end 87.03305 55.706005) (width 0.79) (layer F.Cu) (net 7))
 (segment (start 85.852 55.626) (end 86.953045 55.626) (width 0.79) (layer F.Cu) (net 7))
 (segment (start 99.8474 55.6245) (end 99.8459 55.626) (width 0.35) (layer F.Cu) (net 3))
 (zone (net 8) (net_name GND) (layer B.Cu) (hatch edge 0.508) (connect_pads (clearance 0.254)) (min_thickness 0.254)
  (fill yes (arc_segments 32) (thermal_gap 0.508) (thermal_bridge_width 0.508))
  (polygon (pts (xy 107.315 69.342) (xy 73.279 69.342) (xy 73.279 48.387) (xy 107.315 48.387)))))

